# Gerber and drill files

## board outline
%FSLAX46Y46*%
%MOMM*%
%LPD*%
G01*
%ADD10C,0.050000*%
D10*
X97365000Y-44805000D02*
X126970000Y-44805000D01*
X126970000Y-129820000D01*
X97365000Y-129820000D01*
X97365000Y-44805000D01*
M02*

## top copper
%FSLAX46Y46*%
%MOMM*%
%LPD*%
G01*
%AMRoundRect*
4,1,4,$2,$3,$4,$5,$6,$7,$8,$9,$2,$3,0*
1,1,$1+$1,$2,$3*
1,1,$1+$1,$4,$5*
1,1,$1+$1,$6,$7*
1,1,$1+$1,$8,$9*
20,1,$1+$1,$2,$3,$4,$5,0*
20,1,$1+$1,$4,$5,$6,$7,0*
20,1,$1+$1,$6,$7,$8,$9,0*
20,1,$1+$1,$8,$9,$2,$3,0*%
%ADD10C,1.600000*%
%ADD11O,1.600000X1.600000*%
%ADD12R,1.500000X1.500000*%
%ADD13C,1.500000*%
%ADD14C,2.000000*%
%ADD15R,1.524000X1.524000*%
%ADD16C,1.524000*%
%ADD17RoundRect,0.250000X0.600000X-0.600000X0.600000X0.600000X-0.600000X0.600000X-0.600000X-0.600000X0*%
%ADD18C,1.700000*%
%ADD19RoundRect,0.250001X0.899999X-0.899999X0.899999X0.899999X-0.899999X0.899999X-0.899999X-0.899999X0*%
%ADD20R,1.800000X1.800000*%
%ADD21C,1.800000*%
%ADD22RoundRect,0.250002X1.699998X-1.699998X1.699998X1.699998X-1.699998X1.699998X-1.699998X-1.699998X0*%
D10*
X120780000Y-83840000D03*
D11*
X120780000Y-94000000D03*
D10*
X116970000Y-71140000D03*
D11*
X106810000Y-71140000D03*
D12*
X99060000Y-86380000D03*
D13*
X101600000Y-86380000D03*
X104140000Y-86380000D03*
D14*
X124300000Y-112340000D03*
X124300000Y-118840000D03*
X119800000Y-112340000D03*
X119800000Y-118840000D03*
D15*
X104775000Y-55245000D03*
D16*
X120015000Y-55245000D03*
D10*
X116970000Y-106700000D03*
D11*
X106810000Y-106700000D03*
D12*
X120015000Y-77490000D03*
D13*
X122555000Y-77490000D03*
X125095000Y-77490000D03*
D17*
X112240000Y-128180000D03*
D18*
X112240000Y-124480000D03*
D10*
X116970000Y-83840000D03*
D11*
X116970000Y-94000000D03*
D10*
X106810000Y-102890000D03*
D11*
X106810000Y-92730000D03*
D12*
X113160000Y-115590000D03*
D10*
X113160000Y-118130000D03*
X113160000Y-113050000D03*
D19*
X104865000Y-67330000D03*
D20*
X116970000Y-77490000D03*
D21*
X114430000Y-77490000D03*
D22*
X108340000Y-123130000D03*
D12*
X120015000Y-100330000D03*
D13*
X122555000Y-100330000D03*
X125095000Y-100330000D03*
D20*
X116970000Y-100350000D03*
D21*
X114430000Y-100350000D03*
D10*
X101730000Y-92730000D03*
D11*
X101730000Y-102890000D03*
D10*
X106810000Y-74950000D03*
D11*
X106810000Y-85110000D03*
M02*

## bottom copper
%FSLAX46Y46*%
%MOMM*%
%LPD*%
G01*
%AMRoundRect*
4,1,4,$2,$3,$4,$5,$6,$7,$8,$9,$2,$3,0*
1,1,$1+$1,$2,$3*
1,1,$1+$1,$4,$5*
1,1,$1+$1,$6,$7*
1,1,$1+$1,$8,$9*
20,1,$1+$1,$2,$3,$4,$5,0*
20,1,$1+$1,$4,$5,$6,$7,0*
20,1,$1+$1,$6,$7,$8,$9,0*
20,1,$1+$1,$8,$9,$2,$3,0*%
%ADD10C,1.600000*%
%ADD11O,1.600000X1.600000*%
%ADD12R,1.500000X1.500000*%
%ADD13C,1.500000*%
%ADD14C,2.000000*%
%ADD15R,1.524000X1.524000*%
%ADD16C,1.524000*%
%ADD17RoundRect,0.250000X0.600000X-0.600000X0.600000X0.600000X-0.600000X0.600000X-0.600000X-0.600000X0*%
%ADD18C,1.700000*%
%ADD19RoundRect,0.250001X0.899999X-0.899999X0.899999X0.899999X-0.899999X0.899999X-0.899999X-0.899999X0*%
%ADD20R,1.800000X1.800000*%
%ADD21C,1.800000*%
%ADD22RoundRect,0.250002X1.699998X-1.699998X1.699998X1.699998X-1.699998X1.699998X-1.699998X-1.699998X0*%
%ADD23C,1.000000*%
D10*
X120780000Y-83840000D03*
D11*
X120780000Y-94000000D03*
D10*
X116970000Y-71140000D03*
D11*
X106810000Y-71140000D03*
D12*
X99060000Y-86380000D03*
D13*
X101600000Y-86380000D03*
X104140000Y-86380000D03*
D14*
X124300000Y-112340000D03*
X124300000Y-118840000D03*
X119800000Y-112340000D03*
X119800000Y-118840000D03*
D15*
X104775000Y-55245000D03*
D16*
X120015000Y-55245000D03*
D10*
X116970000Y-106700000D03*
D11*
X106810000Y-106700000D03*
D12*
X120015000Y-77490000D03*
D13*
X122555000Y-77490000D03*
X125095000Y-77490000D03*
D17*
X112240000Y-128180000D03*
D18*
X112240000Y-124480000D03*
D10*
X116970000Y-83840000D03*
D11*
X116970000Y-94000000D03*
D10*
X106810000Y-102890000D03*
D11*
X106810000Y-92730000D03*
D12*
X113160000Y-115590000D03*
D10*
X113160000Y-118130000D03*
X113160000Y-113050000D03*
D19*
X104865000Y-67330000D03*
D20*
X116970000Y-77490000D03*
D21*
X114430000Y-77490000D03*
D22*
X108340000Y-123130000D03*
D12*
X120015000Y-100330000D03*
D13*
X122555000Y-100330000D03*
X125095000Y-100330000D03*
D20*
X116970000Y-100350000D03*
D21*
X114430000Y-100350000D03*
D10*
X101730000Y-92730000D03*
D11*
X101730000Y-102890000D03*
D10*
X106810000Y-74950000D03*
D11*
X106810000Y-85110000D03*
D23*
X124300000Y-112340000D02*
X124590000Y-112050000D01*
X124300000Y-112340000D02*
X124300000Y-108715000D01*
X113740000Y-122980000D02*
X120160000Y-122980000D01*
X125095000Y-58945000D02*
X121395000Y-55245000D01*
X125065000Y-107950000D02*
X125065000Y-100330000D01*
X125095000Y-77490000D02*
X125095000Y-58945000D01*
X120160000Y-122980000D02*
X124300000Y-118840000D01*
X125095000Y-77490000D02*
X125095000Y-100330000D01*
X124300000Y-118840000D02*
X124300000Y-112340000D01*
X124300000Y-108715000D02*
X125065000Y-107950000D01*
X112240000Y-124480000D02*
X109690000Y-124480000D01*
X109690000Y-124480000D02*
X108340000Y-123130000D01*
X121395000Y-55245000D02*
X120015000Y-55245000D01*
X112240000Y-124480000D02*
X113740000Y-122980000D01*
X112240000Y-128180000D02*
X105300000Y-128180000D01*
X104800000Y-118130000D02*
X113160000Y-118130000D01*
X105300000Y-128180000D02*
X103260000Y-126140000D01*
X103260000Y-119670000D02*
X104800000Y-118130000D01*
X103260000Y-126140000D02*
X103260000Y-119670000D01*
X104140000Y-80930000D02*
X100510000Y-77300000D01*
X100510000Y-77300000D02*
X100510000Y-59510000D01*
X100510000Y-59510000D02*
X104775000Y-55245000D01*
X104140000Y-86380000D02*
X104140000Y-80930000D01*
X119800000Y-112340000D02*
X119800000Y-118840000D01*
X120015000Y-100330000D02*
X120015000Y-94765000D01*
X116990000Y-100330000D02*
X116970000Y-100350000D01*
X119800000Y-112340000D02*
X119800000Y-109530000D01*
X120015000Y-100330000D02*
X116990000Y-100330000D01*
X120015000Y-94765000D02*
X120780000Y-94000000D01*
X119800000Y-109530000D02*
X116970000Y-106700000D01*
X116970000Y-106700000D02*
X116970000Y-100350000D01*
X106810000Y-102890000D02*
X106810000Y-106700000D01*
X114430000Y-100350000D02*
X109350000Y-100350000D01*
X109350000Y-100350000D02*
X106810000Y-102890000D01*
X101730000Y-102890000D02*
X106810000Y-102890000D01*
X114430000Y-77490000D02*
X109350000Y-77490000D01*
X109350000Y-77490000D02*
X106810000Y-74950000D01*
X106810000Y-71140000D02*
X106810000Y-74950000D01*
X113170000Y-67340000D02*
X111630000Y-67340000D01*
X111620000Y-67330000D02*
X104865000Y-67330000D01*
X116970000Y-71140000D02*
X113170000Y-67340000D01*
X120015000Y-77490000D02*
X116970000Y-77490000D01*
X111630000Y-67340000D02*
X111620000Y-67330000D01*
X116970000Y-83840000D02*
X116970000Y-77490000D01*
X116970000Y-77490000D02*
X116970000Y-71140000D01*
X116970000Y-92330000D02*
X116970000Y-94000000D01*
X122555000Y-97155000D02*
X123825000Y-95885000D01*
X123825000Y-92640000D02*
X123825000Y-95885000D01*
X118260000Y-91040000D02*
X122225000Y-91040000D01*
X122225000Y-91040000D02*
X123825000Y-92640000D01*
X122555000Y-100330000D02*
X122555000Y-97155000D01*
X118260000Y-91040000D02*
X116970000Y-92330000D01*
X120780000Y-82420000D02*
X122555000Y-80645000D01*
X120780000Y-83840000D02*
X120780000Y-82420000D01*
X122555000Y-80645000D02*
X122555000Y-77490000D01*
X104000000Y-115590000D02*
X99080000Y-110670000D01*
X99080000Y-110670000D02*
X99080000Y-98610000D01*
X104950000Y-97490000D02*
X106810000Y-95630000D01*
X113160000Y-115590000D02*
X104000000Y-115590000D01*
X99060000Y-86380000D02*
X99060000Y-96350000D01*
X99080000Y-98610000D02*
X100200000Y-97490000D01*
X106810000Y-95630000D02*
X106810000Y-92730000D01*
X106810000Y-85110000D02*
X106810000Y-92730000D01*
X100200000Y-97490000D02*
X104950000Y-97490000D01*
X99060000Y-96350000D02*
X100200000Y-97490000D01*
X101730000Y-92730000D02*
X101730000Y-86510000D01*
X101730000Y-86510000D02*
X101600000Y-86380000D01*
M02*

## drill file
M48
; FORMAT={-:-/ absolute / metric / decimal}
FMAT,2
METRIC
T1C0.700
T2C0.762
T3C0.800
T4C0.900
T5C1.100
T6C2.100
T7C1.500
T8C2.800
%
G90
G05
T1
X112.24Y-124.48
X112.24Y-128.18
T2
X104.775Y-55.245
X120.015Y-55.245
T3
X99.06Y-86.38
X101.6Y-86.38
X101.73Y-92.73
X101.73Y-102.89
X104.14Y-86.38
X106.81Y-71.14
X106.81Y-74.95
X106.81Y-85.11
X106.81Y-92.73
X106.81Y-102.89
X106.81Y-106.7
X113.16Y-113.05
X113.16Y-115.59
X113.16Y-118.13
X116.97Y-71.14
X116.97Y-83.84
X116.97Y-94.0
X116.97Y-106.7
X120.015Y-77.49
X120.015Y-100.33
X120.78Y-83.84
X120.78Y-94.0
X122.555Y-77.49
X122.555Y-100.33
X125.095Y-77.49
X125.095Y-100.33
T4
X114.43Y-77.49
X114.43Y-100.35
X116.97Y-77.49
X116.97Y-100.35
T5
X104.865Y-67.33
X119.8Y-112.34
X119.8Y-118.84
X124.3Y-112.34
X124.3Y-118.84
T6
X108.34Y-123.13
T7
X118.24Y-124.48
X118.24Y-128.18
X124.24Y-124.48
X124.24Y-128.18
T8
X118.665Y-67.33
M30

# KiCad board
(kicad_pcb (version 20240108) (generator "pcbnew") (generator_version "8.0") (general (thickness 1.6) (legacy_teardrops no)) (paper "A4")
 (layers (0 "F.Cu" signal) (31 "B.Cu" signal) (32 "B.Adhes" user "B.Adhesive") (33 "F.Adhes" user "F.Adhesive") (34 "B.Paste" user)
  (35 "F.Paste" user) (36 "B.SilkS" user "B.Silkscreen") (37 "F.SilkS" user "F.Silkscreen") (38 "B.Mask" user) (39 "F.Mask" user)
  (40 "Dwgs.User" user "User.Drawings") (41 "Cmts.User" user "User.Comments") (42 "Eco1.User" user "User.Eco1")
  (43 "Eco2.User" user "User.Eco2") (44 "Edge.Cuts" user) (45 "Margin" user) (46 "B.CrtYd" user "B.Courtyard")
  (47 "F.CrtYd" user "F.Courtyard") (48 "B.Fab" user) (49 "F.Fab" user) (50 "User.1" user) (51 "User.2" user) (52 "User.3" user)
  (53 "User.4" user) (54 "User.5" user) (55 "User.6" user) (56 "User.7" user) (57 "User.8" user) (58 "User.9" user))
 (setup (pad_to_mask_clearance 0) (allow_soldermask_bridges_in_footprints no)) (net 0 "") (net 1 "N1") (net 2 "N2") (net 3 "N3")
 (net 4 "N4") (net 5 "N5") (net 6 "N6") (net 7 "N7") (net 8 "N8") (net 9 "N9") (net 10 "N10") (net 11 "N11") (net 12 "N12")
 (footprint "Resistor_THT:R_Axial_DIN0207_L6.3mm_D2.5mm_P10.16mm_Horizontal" (layer "F.Cu") (at 120.78 83.84 -90)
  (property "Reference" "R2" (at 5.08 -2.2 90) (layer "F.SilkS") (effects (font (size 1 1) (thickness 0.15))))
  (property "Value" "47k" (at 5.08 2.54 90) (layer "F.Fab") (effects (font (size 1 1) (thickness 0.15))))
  (pad "1" thru_hole circle (at 0 0 270) (size 1.6 1.6) (drill 0.8) (layers "*.Cu" "*.Mask") (remove_unused_layers no) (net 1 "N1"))
  (pad "2" thru_hole oval (at 10.16 0 270) (size 1.6 1.6) (drill 0.8) (layers "*.Cu" "*.Mask") (remove_unused_layers no) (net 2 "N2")))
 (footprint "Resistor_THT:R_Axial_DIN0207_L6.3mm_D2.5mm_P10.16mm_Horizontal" (layer "F.Cu") (at 116.97 71.14 180)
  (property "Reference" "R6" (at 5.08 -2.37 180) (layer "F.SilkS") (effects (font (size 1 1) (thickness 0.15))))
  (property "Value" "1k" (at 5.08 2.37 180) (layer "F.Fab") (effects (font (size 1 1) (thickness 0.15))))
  (pad "1" thru_hole circle (at 0 0 180) (size 1.6 1.6) (drill 0.8) (layers "*.Cu" "*.Mask") (remove_unused_layers no) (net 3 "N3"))
  (pad "2" thru_hole oval (at 10.16 0 180) (size 1.6 1.6) (drill 0.8) (layers "*.Cu" "*.Mask") (remove_unused_layers no) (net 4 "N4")))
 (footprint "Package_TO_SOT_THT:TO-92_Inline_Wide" (layer "F.Cu") (at 99.06 86.38)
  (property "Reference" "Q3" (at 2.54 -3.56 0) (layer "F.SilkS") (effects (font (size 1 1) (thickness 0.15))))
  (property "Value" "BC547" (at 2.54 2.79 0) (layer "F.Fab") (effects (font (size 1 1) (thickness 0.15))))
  (pad "1" thru_hole rect (at 0 0) (size 1.5 1.5) (drill 0.8) (layers "*.Cu" "*.Mask") (remove_unused_layers no) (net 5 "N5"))
  (pad "2" thru_hole circle (at 2.54 0) (size 1.5 1.5) (drill 0.8) (layers "*.Cu" "*.Mask") (remove_unused_layers no) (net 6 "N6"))
  (pad "3" thru_hole circle (at 5.08 0) (size 1.5 1.5) (drill 0.8) (layers "*.Cu" "*.Mask") (remove_unused_layers no) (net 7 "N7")))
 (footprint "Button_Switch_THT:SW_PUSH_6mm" (layer "F.Cu") (at 124.3 112.34 -90)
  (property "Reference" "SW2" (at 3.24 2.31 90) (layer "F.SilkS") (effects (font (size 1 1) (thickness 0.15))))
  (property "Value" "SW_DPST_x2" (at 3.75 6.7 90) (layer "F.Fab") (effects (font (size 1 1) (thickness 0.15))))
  (pad "1" thru_hole circle (at 0 0) (size 2 2) (drill 1.1) (layers "*.Cu" "*.Mask") (remove_unused_layers no) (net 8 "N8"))
  (pad "1" thru_hole circle (at 6.5 0) (size 2 2) (drill 1.1) (layers "*.Cu" "*.Mask") (remove_unused_layers no) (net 8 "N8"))
  (pad "2" thru_hole circle (at 0 4.5) (size 2 2) (drill 1.1) (layers "*.Cu" "*.Mask") (remove_unused_layers no) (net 2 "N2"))
  (pad "2" thru_hole circle (at 6.5 4.5) (size 2 2) (drill 1.1) (layers "*.Cu" "*.Mask") (remove_unused_layers no) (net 2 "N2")))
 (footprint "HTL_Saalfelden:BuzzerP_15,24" (layer "F.Cu") (at 112.395 55.245)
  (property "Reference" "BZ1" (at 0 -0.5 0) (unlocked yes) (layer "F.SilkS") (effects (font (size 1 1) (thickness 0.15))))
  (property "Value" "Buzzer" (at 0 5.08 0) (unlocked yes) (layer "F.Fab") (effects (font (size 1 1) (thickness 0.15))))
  (pad "1" thru_hole rect (at -7.62 0) (size 1.524 1.524) (drill 0.762) (layers "*.Cu" "*.Mask") (remove_unused_layers no) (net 7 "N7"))
  (pad "2" thru_hole circle (at 7.62 0) (size 1.524 1.524) (drill 0.762) (layers "*.Cu" "*.Mask") (remove_unused_layers no) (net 8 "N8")))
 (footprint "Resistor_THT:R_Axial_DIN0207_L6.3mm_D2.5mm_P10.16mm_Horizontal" (layer "F.Cu") (at 116.97 106.7 180)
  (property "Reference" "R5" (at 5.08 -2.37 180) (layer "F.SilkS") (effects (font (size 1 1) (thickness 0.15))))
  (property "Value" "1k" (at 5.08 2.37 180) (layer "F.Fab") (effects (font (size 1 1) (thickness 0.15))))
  (pad "1" thru_hole circle (at 0 0 180) (size 1.6 1.6) (drill 0.8) (layers "*.Cu" "*.Mask") (remove_unused_layers no) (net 2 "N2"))
  (pad "2" thru_hole oval (at 10.16 0 180) (size 1.6 1.6) (drill 0.8) (layers "*.Cu" "*.Mask") (remove_unused_layers no) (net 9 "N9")))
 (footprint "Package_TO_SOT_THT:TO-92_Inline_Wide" (layer "F.Cu") (at 120.015 77.49)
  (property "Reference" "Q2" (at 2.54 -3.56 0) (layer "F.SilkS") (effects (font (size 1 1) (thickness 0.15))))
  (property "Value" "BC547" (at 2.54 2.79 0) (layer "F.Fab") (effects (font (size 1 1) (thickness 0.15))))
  (pad "1" thru_hole rect (at 0 0) (size 1.5 1.5) (drill 0.8) (layers "*.Cu" "*.Mask") (remove_unused_layers no) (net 3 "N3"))
  (pad "2" thru_hole circle (at 2.54 0) (size 1.5 1.5) (drill 0.8) (layers "*.Cu" "*.Mask") (remove_unused_layers no) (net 1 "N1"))
  (pad "3" thru_hole circle (at 5.08 0) (size 1.5 1.5) (drill 0.8) (layers "*.Cu" "*.Mask") (remove_unused_layers no) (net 8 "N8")))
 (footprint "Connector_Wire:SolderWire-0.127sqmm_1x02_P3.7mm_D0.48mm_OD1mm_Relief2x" (layer "F.Cu") (at 112.24 128.18 90)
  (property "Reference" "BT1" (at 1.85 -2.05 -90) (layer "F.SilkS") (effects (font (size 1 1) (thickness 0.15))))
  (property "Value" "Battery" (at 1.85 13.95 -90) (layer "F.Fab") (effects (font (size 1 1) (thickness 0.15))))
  (pad "" np_thru_hole circle (at 0 6 90) (size 1.5 1.5) (drill 1.5) (layers "*.Cu" "*.Mask"))
  (pad "" np_thru_hole circle (at 0 12 90) (size 1.5 1.5) (drill 1.5) (layers "*.Cu" "*.Mask"))
  (pad "" np_thru_hole circle (at 3.7 6 90) (size 1.5 1.5) (drill 1.5) (layers "*.Cu" "*.Mask"))
  (pad "" np_thru_hole circle (at 3.7 12 90) (size 1.5 1.5) (drill 1.5) (layers "*.Cu" "*.Mask"))
  (pad "1" thru_hole roundrect (at 0 0 90) (size 1.7 1.7) (drill 0.7) (layers "*.Cu" "*.Mask") (remove_unused_layers no)
   (roundrect_rratio 0.147059) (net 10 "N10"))
  (pad "2" thru_hole circle (at 3.7 0 90) (size 1.7 1.7) (drill 0.7) (layers "*.Cu" "*.Mask") (remove_unused_layers no) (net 8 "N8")))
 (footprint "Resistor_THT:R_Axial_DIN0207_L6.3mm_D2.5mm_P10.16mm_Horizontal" (layer "F.Cu") (at 116.97 83.84 -90)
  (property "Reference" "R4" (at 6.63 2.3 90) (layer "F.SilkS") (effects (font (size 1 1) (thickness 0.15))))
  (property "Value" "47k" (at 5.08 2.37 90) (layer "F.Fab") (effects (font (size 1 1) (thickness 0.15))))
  (pad "1" thru_hole circle (at 0 0 270) (size 1.6 1.6) (drill 0.8) (layers "*.Cu" "*.Mask") (remove_unused_layers no) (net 3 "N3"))
  (pad "2" thru_hole oval (at 10.16 0 270) (size 1.6 1.6) (drill 0.8) (layers "*.Cu" "*.Mask") (remove_unused_layers no) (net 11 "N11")))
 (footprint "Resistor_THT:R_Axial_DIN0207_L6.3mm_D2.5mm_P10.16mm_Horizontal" (layer "F.Cu") (at 106.81 102.89 90)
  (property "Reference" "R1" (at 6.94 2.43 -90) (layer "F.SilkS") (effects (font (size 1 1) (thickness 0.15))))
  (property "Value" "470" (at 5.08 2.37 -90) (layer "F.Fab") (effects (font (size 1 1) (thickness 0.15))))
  (pad "1" thru_hole circle (at 0 0 90) (size 1.6 1.6) (drill 0.8) (layers "*.Cu" "*.Mask") (remove_unused_layers no) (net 9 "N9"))
  (pad "2" thru_hole oval (at 10.16 0 90) (size 1.6 1.6) (drill 0.8) (layers "*.Cu" "*.Mask") (remove_unused_layers no) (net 5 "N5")))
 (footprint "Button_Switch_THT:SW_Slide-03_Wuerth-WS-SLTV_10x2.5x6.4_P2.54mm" (layer "F.Cu") (at 113.16 115.59 90)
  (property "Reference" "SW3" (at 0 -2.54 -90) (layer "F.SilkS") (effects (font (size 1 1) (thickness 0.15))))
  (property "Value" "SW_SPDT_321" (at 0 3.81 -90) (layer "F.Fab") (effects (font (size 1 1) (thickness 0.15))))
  (pad "1" thru_hole rect (at 0 0 90) (size 1.5 1.5) (drill 0.8) (layers "*.Cu" "*.Mask") (remove_unused_layers no) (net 5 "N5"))
  (pad "2" thru_hole circle (at -2.54 0 90) (size 1.6 1.6) (drill 0.8) (layers "*.Cu" "*.Mask") (remove_unused_layers no) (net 10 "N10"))
  (pad "3" thru_hole circle (at 2.54 0 90) (size 1.6 1.6) (drill 0.8) (layers "*.Cu" "*.Mask") (remove_unused_layers no) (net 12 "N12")))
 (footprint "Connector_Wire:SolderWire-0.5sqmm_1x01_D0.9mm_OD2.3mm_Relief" (layer "F.Cu") (at 104.865 67.33 90)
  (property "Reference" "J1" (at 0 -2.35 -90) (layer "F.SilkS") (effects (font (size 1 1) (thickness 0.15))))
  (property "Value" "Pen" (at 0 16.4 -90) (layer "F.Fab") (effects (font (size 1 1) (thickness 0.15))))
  (pad "" np_thru_hole circle (at 0 13.8 90) (size 2.8 2.8) (drill 2.8) (layers "*.Cu" "*.Mask"))
  (pad "1" thru_hole roundrect (at 0 0 90) (size 2.3 2.3) (drill 1.1) (layers "*.Cu" "*.Mask") (remove_unused_layers no)
   (roundrect_rratio 0.108696) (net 3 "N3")))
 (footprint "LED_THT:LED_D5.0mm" (layer "F.Cu") (at 116.97 77.49 180)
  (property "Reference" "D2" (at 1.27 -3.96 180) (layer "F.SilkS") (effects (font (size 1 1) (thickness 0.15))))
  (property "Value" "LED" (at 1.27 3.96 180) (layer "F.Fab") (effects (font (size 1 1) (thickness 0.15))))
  (pad "1" thru_hole rect (at 0 0 180) (size 1.8 1.8) (drill 0.9) (layers "*.Cu" "*.Mask") (remove_unused_layers no) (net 3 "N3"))
  (pad "2" thru_hole circle (at 2.54 0 180) (size 1.8 1.8) (drill 0.9) (layers "*.Cu" "*.Mask") (remove_unused_layers no) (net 4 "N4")))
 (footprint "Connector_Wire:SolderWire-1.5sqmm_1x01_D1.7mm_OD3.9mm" (layer "F.Cu") (at 108.34 123.13 90)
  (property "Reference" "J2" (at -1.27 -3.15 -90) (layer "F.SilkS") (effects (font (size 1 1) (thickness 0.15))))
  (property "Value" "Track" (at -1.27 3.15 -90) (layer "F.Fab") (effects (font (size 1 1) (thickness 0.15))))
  (pad "1" thru_hole roundrect (at 0 0 90) (size 3.9 3.9) (drill 2.1) (layers "*.Cu" "*.Mask") (remove_unused_layers no)
   (roundrect_rratio 0.064103) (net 8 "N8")))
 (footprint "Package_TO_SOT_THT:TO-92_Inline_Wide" (layer "F.Cu") (at 120.015 100.33)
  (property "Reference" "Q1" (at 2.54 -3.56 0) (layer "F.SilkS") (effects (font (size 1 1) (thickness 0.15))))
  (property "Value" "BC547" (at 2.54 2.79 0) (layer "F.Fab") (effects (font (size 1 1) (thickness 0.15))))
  (pad "1" thru_hole rect (at 0 0) (size 1.5 1.5) (drill 0.8) (layers "*.Cu" "*.Mask") (remove_unused_layers no) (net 2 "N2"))
  (pad "2" thru_hole circle (at 2.54 0) (size 1.5 1.5) (drill 0.8) (layers "*.Cu" "*.Mask") (remove_unused_layers no) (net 11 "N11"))
  (pad "3" thru_hole circle (at 5.08 0) (size 1.5 1.5) (drill 0.8) (layers "*.Cu" "*.Mask") (remove_unused_layers no) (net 8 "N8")))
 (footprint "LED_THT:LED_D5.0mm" (layer "F.Cu") (at 116.97 100.35 180)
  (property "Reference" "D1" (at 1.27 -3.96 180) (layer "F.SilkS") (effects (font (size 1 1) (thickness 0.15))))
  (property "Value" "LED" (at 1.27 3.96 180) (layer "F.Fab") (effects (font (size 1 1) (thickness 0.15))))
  (pad "1" thru_hole rect (at 0 0 180) (size 1.8 1.8) (drill 0.9) (layers "*.Cu" "*.Mask") (remove_unused_layers no) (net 2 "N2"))
  (pad "2" thru_hole circle (at 2.54 0 180) (size 1.8 1.8) (drill 0.9) (layers "*.Cu" "*.Mask") (remove_unused_layers no) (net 9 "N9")))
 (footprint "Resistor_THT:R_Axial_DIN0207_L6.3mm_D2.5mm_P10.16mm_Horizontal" (layer "F.Cu") (at 101.73 92.73 -90)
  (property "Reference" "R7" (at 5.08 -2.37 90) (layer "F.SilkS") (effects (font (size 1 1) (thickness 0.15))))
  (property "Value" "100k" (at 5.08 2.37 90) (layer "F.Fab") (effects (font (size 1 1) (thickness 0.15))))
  (pad "1" thru_hole circle (at 0 0 270) (size 1.6 1.6) (drill 0.8) (layers "*.Cu" "*.Mask") (remove_unused_layers no) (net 6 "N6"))
  (pad "2" thru_hole oval (at 10.16 0 270) (size 1.6 1.6) (drill 0.8) (layers "*.Cu" "*.Mask") (remove_unused_layers no) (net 9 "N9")))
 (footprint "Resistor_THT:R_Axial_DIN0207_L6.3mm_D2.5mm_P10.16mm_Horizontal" (layer "F.Cu") (at 106.81 74.95 -90)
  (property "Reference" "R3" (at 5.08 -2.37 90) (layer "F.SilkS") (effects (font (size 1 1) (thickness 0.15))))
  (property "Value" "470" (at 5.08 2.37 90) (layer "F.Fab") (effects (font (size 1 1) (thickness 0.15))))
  (pad "1" thru_hole circle (at 0 0 270) (size 1.6 1.6) (drill 0.8) (layers "*.Cu" "*.Mask") (remove_unused_layers no) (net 4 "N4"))
  (pad "2" thru_hole oval (at 10.16 0 270) (size 1.6 1.6) (drill 0.8) (layers "*.Cu" "*.Mask") (remove_unused_layers no) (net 5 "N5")))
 (gr_rect (start 97.365 44.805) (end 126.97 129.82) (stroke (width 0.05) (type default)) (fill none) (layer "Edge.Cuts"))
 (segment (start 124.3 112.34) (end 124.59 112.05) (width 1) (layer "B.Cu") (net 8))
 (segment (start 124.3 112.34) (end 124.3 108.715) (width 1) (layer "B.Cu") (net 8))
 (segment (start 113.74 122.98) (end 120.16 122.98) (width 1) (layer "B.Cu") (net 8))
 (segment (start 125.095 58.945) (end 121.395 55.245) (width 1) (layer "B.Cu") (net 8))
 (segment (start 125.065 107.95) (end 125.065 100.33) (width 1) (layer "B.Cu") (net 8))
 (segment (start 125.095 77.49) (end 125.095 58.945) (width 1) (layer "B.Cu") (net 8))
 (segment (start 120.16 122.98) (end 124.3 118.84) (width 1) (layer "B.Cu") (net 8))
 (segment (start 125.095 77.49) (end 125.095 100.33) (width 1) (layer "B.Cu") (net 8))
 (segment (start 124.3 118.84) (end 124.3 112.34) (width 1) (layer "B.Cu") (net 8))
 (segment (start 124.3 108.715) (end 125.065 107.95) (width 1) (layer "B.Cu") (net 8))
 (segment (start 112.24 124.48) (end 109.69 124.48) (width 1) (layer "B.Cu") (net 8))
 (segment (start 109.69 124.48) (end 108.34 123.13) (width 1) (layer "B.Cu") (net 8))
 (segment (start 121.395 55.245) (end 120.015 55.245) (width 1) (layer "B.Cu") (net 8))
 (segment (start 112.24 124.48) (end 113.74 122.98) (width 1) (layer "B.Cu") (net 8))
 (segment (start 112.24 128.18) (end 105.3 128.18) (width 1) (layer "B.Cu") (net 10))
 (segment (start 104.8 118.13) (end 113.16 118.13) (width 1) (layer "B.Cu") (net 10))
 (segment (start 105.3 128.18) (end 103.26 126.14) (width 1) (layer "B.Cu") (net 10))
 (segment (start 103.26 119.67) (end 104.8 118.13) (width 1) (layer "B.Cu") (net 10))
 (segment (start 103.26 126.14) (end 103.26 119.67) (width 1) (layer "B.Cu") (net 10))
 (segment (start 104.14 80.93) (end 100.51 77.3) (width 1) (layer "B.Cu") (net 7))
 (segment (start 100.51 77.3) (end 100.51 59.51) (width 1) (layer "B.Cu") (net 7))
 (segment (start 100.51 59.51) (end 104.775 55.245) (width 1) (layer "B.Cu") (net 7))
 (segment (start 104.14 86.38) (end 104.14 80.93) (width 1) (layer "B.Cu") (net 7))
 (segment (start 119.8 112.34) (end 119.8 118.84) (width 1) (layer "B.Cu") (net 2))
 (segment (start 120.015 100.33) (end 120.015 94.765) (width 1) (layer "B.Cu") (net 2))
 (segment (start 116.99 100.33) (end 116.97 100.35) (width 1) (layer "B.Cu") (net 2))
 (segment (start 119.8 112.34) (end 119.8 109.53) (width 1) (layer "B.Cu") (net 2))
 (segment (start 120.015 100.33) (end 116.99 100.33) (width 1) (layer "B.Cu") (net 2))
 (segment (start 120.015 94.765) (end 120.78 94) (width 1) (layer "B.Cu") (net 2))
 (segment (start 119.8 109.53) (end 116.97 106.7) (width 1) (layer "B.Cu") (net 2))
 (segment (start 116.97 106.7) (end 116.97 100.35) (width 1) (layer "B.Cu") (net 2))
 (segment (start 106.81 102.89) (end 106.81 106.7) (width 1) (layer "B.Cu") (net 9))
 (segment (start 114.43 100.35) (end 109.35 100.35) (width 1) (layer "B.Cu") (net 9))
 (segment (start 109.35 100.35) (end 106.81 102.89) (width 1) (layer "B.Cu") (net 9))
 (segment (start 101.73 102.89) (end 106.81 102.89) (width 1) (layer "B.Cu") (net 9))
 (segment (start 114.43 77.49) (end 109.35 77.49) (width 1) (layer "B.Cu") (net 4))
 (segment (start 109.35 77.49) (end 106.81 74.95) (width 1) (layer "B.Cu") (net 4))
 (segment (start 106.81 71.14) (end 106.81 74.95) (width 1) (layer "B.Cu") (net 4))
 (segment (start 113.17 67.34) (end 111.63 67.34) (width 1) (layer "B.Cu") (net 3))
 (segment (start 111.62 67.33) (end 104.865 67.33) (width 1) (layer "B.Cu") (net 3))
 (segment (start 116.97 71.14) (end 113.17 67.34) (width 1) (layer "B.Cu") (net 3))
 (segment (start 120.015 77.49) (end 116.97 77.49) (width 1) (layer "B.Cu") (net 3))
 (segment (start 111.63 67.34) (end 111.62 67.33) (width 1) (layer "B.Cu") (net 3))
 (segment (start 116.97 83.84) (end 116.97 77.49) (width 1) (layer "B.Cu") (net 3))
 (segment (start 116.97 77.49) (end 116.97 71.14) (width 1) (layer "B.Cu") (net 3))
 (segment (start 116.97 92.33) (end 116.97 94) (width 1) (layer "B.Cu") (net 11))
 (segment (start 122.555 97.155) (end 123.825 95.885) (width 1) (layer "B.Cu") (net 11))
 (segment (start 123.825 92.64) (end 123.825 95.885) (width 1) (layer "B.Cu") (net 11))
 (segment (start 118.26 91.04) (end 122.225 91.04) (width 1) (layer "B.Cu") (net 11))
 (segment (start 122.225 91.04) (end 123.825 92.64) (width 1) (layer "B.Cu") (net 11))
 (segment (start 122.555 100.33) (end 122.555 97.155) (width 1) (layer "B.Cu") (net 11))
 (segment (start 118.26 91.04) (end 116.97 92.33) (width 1) (layer "B.Cu") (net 11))
 (segment (start 120.78 82.42) (end 122.555 80.645) (width 1) (layer "B.Cu") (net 1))
 (segment (start 120.78 83.84) (end 120.78 82.42) (width 1) (layer "B.Cu") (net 1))
 (segment (start 122.555 80.645) (end 122.555 77.49) (width 1) (layer "B.Cu") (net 1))
 (segment (start 104 115.59) (end 99.08 110.67) (width 1) (layer "B.Cu") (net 5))
 (segment (start 99.08 110.67) (end 99.08 98.61) (width 1) (layer "B.Cu") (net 5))
 (segment (start 104.95 97.49) (end 106.81 95.63) (width 1) (layer "B.Cu") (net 5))
 (segment (start 113.16 115.59) (end 104 115.59) (width 1) (layer "B.Cu") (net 5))
 (segment (start 99.06 86.38) (end 99.06 96.35) (width 1) (layer "B.Cu") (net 5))
 (segment (start 99.08 98.61) (end 100.2 97.49) (width 1) (layer "B.Cu") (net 5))
 (segment (start 106.81 95.63) (end 106.81 92.73) (width 1) (layer "B.Cu") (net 5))
 (segment (start 106.81 85.11) (end 106.81 92.73) (width 1) (layer "B.Cu") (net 5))
 (segment (start 100.2 97.49) (end 104.95 97.49) (width 1) (layer "B.Cu") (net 5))
 (segment (start 99.06 96.35) (end 100.2 97.49) (width 1) (layer "B.Cu") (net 5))
 (segment (start 101.73 92.73) (end 101.73 86.51) (width 1) (layer "B.Cu") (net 6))
 (segment (start 101.73 86.51) (end 101.6 86.38) (width 1) (layer "B.Cu") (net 6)))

